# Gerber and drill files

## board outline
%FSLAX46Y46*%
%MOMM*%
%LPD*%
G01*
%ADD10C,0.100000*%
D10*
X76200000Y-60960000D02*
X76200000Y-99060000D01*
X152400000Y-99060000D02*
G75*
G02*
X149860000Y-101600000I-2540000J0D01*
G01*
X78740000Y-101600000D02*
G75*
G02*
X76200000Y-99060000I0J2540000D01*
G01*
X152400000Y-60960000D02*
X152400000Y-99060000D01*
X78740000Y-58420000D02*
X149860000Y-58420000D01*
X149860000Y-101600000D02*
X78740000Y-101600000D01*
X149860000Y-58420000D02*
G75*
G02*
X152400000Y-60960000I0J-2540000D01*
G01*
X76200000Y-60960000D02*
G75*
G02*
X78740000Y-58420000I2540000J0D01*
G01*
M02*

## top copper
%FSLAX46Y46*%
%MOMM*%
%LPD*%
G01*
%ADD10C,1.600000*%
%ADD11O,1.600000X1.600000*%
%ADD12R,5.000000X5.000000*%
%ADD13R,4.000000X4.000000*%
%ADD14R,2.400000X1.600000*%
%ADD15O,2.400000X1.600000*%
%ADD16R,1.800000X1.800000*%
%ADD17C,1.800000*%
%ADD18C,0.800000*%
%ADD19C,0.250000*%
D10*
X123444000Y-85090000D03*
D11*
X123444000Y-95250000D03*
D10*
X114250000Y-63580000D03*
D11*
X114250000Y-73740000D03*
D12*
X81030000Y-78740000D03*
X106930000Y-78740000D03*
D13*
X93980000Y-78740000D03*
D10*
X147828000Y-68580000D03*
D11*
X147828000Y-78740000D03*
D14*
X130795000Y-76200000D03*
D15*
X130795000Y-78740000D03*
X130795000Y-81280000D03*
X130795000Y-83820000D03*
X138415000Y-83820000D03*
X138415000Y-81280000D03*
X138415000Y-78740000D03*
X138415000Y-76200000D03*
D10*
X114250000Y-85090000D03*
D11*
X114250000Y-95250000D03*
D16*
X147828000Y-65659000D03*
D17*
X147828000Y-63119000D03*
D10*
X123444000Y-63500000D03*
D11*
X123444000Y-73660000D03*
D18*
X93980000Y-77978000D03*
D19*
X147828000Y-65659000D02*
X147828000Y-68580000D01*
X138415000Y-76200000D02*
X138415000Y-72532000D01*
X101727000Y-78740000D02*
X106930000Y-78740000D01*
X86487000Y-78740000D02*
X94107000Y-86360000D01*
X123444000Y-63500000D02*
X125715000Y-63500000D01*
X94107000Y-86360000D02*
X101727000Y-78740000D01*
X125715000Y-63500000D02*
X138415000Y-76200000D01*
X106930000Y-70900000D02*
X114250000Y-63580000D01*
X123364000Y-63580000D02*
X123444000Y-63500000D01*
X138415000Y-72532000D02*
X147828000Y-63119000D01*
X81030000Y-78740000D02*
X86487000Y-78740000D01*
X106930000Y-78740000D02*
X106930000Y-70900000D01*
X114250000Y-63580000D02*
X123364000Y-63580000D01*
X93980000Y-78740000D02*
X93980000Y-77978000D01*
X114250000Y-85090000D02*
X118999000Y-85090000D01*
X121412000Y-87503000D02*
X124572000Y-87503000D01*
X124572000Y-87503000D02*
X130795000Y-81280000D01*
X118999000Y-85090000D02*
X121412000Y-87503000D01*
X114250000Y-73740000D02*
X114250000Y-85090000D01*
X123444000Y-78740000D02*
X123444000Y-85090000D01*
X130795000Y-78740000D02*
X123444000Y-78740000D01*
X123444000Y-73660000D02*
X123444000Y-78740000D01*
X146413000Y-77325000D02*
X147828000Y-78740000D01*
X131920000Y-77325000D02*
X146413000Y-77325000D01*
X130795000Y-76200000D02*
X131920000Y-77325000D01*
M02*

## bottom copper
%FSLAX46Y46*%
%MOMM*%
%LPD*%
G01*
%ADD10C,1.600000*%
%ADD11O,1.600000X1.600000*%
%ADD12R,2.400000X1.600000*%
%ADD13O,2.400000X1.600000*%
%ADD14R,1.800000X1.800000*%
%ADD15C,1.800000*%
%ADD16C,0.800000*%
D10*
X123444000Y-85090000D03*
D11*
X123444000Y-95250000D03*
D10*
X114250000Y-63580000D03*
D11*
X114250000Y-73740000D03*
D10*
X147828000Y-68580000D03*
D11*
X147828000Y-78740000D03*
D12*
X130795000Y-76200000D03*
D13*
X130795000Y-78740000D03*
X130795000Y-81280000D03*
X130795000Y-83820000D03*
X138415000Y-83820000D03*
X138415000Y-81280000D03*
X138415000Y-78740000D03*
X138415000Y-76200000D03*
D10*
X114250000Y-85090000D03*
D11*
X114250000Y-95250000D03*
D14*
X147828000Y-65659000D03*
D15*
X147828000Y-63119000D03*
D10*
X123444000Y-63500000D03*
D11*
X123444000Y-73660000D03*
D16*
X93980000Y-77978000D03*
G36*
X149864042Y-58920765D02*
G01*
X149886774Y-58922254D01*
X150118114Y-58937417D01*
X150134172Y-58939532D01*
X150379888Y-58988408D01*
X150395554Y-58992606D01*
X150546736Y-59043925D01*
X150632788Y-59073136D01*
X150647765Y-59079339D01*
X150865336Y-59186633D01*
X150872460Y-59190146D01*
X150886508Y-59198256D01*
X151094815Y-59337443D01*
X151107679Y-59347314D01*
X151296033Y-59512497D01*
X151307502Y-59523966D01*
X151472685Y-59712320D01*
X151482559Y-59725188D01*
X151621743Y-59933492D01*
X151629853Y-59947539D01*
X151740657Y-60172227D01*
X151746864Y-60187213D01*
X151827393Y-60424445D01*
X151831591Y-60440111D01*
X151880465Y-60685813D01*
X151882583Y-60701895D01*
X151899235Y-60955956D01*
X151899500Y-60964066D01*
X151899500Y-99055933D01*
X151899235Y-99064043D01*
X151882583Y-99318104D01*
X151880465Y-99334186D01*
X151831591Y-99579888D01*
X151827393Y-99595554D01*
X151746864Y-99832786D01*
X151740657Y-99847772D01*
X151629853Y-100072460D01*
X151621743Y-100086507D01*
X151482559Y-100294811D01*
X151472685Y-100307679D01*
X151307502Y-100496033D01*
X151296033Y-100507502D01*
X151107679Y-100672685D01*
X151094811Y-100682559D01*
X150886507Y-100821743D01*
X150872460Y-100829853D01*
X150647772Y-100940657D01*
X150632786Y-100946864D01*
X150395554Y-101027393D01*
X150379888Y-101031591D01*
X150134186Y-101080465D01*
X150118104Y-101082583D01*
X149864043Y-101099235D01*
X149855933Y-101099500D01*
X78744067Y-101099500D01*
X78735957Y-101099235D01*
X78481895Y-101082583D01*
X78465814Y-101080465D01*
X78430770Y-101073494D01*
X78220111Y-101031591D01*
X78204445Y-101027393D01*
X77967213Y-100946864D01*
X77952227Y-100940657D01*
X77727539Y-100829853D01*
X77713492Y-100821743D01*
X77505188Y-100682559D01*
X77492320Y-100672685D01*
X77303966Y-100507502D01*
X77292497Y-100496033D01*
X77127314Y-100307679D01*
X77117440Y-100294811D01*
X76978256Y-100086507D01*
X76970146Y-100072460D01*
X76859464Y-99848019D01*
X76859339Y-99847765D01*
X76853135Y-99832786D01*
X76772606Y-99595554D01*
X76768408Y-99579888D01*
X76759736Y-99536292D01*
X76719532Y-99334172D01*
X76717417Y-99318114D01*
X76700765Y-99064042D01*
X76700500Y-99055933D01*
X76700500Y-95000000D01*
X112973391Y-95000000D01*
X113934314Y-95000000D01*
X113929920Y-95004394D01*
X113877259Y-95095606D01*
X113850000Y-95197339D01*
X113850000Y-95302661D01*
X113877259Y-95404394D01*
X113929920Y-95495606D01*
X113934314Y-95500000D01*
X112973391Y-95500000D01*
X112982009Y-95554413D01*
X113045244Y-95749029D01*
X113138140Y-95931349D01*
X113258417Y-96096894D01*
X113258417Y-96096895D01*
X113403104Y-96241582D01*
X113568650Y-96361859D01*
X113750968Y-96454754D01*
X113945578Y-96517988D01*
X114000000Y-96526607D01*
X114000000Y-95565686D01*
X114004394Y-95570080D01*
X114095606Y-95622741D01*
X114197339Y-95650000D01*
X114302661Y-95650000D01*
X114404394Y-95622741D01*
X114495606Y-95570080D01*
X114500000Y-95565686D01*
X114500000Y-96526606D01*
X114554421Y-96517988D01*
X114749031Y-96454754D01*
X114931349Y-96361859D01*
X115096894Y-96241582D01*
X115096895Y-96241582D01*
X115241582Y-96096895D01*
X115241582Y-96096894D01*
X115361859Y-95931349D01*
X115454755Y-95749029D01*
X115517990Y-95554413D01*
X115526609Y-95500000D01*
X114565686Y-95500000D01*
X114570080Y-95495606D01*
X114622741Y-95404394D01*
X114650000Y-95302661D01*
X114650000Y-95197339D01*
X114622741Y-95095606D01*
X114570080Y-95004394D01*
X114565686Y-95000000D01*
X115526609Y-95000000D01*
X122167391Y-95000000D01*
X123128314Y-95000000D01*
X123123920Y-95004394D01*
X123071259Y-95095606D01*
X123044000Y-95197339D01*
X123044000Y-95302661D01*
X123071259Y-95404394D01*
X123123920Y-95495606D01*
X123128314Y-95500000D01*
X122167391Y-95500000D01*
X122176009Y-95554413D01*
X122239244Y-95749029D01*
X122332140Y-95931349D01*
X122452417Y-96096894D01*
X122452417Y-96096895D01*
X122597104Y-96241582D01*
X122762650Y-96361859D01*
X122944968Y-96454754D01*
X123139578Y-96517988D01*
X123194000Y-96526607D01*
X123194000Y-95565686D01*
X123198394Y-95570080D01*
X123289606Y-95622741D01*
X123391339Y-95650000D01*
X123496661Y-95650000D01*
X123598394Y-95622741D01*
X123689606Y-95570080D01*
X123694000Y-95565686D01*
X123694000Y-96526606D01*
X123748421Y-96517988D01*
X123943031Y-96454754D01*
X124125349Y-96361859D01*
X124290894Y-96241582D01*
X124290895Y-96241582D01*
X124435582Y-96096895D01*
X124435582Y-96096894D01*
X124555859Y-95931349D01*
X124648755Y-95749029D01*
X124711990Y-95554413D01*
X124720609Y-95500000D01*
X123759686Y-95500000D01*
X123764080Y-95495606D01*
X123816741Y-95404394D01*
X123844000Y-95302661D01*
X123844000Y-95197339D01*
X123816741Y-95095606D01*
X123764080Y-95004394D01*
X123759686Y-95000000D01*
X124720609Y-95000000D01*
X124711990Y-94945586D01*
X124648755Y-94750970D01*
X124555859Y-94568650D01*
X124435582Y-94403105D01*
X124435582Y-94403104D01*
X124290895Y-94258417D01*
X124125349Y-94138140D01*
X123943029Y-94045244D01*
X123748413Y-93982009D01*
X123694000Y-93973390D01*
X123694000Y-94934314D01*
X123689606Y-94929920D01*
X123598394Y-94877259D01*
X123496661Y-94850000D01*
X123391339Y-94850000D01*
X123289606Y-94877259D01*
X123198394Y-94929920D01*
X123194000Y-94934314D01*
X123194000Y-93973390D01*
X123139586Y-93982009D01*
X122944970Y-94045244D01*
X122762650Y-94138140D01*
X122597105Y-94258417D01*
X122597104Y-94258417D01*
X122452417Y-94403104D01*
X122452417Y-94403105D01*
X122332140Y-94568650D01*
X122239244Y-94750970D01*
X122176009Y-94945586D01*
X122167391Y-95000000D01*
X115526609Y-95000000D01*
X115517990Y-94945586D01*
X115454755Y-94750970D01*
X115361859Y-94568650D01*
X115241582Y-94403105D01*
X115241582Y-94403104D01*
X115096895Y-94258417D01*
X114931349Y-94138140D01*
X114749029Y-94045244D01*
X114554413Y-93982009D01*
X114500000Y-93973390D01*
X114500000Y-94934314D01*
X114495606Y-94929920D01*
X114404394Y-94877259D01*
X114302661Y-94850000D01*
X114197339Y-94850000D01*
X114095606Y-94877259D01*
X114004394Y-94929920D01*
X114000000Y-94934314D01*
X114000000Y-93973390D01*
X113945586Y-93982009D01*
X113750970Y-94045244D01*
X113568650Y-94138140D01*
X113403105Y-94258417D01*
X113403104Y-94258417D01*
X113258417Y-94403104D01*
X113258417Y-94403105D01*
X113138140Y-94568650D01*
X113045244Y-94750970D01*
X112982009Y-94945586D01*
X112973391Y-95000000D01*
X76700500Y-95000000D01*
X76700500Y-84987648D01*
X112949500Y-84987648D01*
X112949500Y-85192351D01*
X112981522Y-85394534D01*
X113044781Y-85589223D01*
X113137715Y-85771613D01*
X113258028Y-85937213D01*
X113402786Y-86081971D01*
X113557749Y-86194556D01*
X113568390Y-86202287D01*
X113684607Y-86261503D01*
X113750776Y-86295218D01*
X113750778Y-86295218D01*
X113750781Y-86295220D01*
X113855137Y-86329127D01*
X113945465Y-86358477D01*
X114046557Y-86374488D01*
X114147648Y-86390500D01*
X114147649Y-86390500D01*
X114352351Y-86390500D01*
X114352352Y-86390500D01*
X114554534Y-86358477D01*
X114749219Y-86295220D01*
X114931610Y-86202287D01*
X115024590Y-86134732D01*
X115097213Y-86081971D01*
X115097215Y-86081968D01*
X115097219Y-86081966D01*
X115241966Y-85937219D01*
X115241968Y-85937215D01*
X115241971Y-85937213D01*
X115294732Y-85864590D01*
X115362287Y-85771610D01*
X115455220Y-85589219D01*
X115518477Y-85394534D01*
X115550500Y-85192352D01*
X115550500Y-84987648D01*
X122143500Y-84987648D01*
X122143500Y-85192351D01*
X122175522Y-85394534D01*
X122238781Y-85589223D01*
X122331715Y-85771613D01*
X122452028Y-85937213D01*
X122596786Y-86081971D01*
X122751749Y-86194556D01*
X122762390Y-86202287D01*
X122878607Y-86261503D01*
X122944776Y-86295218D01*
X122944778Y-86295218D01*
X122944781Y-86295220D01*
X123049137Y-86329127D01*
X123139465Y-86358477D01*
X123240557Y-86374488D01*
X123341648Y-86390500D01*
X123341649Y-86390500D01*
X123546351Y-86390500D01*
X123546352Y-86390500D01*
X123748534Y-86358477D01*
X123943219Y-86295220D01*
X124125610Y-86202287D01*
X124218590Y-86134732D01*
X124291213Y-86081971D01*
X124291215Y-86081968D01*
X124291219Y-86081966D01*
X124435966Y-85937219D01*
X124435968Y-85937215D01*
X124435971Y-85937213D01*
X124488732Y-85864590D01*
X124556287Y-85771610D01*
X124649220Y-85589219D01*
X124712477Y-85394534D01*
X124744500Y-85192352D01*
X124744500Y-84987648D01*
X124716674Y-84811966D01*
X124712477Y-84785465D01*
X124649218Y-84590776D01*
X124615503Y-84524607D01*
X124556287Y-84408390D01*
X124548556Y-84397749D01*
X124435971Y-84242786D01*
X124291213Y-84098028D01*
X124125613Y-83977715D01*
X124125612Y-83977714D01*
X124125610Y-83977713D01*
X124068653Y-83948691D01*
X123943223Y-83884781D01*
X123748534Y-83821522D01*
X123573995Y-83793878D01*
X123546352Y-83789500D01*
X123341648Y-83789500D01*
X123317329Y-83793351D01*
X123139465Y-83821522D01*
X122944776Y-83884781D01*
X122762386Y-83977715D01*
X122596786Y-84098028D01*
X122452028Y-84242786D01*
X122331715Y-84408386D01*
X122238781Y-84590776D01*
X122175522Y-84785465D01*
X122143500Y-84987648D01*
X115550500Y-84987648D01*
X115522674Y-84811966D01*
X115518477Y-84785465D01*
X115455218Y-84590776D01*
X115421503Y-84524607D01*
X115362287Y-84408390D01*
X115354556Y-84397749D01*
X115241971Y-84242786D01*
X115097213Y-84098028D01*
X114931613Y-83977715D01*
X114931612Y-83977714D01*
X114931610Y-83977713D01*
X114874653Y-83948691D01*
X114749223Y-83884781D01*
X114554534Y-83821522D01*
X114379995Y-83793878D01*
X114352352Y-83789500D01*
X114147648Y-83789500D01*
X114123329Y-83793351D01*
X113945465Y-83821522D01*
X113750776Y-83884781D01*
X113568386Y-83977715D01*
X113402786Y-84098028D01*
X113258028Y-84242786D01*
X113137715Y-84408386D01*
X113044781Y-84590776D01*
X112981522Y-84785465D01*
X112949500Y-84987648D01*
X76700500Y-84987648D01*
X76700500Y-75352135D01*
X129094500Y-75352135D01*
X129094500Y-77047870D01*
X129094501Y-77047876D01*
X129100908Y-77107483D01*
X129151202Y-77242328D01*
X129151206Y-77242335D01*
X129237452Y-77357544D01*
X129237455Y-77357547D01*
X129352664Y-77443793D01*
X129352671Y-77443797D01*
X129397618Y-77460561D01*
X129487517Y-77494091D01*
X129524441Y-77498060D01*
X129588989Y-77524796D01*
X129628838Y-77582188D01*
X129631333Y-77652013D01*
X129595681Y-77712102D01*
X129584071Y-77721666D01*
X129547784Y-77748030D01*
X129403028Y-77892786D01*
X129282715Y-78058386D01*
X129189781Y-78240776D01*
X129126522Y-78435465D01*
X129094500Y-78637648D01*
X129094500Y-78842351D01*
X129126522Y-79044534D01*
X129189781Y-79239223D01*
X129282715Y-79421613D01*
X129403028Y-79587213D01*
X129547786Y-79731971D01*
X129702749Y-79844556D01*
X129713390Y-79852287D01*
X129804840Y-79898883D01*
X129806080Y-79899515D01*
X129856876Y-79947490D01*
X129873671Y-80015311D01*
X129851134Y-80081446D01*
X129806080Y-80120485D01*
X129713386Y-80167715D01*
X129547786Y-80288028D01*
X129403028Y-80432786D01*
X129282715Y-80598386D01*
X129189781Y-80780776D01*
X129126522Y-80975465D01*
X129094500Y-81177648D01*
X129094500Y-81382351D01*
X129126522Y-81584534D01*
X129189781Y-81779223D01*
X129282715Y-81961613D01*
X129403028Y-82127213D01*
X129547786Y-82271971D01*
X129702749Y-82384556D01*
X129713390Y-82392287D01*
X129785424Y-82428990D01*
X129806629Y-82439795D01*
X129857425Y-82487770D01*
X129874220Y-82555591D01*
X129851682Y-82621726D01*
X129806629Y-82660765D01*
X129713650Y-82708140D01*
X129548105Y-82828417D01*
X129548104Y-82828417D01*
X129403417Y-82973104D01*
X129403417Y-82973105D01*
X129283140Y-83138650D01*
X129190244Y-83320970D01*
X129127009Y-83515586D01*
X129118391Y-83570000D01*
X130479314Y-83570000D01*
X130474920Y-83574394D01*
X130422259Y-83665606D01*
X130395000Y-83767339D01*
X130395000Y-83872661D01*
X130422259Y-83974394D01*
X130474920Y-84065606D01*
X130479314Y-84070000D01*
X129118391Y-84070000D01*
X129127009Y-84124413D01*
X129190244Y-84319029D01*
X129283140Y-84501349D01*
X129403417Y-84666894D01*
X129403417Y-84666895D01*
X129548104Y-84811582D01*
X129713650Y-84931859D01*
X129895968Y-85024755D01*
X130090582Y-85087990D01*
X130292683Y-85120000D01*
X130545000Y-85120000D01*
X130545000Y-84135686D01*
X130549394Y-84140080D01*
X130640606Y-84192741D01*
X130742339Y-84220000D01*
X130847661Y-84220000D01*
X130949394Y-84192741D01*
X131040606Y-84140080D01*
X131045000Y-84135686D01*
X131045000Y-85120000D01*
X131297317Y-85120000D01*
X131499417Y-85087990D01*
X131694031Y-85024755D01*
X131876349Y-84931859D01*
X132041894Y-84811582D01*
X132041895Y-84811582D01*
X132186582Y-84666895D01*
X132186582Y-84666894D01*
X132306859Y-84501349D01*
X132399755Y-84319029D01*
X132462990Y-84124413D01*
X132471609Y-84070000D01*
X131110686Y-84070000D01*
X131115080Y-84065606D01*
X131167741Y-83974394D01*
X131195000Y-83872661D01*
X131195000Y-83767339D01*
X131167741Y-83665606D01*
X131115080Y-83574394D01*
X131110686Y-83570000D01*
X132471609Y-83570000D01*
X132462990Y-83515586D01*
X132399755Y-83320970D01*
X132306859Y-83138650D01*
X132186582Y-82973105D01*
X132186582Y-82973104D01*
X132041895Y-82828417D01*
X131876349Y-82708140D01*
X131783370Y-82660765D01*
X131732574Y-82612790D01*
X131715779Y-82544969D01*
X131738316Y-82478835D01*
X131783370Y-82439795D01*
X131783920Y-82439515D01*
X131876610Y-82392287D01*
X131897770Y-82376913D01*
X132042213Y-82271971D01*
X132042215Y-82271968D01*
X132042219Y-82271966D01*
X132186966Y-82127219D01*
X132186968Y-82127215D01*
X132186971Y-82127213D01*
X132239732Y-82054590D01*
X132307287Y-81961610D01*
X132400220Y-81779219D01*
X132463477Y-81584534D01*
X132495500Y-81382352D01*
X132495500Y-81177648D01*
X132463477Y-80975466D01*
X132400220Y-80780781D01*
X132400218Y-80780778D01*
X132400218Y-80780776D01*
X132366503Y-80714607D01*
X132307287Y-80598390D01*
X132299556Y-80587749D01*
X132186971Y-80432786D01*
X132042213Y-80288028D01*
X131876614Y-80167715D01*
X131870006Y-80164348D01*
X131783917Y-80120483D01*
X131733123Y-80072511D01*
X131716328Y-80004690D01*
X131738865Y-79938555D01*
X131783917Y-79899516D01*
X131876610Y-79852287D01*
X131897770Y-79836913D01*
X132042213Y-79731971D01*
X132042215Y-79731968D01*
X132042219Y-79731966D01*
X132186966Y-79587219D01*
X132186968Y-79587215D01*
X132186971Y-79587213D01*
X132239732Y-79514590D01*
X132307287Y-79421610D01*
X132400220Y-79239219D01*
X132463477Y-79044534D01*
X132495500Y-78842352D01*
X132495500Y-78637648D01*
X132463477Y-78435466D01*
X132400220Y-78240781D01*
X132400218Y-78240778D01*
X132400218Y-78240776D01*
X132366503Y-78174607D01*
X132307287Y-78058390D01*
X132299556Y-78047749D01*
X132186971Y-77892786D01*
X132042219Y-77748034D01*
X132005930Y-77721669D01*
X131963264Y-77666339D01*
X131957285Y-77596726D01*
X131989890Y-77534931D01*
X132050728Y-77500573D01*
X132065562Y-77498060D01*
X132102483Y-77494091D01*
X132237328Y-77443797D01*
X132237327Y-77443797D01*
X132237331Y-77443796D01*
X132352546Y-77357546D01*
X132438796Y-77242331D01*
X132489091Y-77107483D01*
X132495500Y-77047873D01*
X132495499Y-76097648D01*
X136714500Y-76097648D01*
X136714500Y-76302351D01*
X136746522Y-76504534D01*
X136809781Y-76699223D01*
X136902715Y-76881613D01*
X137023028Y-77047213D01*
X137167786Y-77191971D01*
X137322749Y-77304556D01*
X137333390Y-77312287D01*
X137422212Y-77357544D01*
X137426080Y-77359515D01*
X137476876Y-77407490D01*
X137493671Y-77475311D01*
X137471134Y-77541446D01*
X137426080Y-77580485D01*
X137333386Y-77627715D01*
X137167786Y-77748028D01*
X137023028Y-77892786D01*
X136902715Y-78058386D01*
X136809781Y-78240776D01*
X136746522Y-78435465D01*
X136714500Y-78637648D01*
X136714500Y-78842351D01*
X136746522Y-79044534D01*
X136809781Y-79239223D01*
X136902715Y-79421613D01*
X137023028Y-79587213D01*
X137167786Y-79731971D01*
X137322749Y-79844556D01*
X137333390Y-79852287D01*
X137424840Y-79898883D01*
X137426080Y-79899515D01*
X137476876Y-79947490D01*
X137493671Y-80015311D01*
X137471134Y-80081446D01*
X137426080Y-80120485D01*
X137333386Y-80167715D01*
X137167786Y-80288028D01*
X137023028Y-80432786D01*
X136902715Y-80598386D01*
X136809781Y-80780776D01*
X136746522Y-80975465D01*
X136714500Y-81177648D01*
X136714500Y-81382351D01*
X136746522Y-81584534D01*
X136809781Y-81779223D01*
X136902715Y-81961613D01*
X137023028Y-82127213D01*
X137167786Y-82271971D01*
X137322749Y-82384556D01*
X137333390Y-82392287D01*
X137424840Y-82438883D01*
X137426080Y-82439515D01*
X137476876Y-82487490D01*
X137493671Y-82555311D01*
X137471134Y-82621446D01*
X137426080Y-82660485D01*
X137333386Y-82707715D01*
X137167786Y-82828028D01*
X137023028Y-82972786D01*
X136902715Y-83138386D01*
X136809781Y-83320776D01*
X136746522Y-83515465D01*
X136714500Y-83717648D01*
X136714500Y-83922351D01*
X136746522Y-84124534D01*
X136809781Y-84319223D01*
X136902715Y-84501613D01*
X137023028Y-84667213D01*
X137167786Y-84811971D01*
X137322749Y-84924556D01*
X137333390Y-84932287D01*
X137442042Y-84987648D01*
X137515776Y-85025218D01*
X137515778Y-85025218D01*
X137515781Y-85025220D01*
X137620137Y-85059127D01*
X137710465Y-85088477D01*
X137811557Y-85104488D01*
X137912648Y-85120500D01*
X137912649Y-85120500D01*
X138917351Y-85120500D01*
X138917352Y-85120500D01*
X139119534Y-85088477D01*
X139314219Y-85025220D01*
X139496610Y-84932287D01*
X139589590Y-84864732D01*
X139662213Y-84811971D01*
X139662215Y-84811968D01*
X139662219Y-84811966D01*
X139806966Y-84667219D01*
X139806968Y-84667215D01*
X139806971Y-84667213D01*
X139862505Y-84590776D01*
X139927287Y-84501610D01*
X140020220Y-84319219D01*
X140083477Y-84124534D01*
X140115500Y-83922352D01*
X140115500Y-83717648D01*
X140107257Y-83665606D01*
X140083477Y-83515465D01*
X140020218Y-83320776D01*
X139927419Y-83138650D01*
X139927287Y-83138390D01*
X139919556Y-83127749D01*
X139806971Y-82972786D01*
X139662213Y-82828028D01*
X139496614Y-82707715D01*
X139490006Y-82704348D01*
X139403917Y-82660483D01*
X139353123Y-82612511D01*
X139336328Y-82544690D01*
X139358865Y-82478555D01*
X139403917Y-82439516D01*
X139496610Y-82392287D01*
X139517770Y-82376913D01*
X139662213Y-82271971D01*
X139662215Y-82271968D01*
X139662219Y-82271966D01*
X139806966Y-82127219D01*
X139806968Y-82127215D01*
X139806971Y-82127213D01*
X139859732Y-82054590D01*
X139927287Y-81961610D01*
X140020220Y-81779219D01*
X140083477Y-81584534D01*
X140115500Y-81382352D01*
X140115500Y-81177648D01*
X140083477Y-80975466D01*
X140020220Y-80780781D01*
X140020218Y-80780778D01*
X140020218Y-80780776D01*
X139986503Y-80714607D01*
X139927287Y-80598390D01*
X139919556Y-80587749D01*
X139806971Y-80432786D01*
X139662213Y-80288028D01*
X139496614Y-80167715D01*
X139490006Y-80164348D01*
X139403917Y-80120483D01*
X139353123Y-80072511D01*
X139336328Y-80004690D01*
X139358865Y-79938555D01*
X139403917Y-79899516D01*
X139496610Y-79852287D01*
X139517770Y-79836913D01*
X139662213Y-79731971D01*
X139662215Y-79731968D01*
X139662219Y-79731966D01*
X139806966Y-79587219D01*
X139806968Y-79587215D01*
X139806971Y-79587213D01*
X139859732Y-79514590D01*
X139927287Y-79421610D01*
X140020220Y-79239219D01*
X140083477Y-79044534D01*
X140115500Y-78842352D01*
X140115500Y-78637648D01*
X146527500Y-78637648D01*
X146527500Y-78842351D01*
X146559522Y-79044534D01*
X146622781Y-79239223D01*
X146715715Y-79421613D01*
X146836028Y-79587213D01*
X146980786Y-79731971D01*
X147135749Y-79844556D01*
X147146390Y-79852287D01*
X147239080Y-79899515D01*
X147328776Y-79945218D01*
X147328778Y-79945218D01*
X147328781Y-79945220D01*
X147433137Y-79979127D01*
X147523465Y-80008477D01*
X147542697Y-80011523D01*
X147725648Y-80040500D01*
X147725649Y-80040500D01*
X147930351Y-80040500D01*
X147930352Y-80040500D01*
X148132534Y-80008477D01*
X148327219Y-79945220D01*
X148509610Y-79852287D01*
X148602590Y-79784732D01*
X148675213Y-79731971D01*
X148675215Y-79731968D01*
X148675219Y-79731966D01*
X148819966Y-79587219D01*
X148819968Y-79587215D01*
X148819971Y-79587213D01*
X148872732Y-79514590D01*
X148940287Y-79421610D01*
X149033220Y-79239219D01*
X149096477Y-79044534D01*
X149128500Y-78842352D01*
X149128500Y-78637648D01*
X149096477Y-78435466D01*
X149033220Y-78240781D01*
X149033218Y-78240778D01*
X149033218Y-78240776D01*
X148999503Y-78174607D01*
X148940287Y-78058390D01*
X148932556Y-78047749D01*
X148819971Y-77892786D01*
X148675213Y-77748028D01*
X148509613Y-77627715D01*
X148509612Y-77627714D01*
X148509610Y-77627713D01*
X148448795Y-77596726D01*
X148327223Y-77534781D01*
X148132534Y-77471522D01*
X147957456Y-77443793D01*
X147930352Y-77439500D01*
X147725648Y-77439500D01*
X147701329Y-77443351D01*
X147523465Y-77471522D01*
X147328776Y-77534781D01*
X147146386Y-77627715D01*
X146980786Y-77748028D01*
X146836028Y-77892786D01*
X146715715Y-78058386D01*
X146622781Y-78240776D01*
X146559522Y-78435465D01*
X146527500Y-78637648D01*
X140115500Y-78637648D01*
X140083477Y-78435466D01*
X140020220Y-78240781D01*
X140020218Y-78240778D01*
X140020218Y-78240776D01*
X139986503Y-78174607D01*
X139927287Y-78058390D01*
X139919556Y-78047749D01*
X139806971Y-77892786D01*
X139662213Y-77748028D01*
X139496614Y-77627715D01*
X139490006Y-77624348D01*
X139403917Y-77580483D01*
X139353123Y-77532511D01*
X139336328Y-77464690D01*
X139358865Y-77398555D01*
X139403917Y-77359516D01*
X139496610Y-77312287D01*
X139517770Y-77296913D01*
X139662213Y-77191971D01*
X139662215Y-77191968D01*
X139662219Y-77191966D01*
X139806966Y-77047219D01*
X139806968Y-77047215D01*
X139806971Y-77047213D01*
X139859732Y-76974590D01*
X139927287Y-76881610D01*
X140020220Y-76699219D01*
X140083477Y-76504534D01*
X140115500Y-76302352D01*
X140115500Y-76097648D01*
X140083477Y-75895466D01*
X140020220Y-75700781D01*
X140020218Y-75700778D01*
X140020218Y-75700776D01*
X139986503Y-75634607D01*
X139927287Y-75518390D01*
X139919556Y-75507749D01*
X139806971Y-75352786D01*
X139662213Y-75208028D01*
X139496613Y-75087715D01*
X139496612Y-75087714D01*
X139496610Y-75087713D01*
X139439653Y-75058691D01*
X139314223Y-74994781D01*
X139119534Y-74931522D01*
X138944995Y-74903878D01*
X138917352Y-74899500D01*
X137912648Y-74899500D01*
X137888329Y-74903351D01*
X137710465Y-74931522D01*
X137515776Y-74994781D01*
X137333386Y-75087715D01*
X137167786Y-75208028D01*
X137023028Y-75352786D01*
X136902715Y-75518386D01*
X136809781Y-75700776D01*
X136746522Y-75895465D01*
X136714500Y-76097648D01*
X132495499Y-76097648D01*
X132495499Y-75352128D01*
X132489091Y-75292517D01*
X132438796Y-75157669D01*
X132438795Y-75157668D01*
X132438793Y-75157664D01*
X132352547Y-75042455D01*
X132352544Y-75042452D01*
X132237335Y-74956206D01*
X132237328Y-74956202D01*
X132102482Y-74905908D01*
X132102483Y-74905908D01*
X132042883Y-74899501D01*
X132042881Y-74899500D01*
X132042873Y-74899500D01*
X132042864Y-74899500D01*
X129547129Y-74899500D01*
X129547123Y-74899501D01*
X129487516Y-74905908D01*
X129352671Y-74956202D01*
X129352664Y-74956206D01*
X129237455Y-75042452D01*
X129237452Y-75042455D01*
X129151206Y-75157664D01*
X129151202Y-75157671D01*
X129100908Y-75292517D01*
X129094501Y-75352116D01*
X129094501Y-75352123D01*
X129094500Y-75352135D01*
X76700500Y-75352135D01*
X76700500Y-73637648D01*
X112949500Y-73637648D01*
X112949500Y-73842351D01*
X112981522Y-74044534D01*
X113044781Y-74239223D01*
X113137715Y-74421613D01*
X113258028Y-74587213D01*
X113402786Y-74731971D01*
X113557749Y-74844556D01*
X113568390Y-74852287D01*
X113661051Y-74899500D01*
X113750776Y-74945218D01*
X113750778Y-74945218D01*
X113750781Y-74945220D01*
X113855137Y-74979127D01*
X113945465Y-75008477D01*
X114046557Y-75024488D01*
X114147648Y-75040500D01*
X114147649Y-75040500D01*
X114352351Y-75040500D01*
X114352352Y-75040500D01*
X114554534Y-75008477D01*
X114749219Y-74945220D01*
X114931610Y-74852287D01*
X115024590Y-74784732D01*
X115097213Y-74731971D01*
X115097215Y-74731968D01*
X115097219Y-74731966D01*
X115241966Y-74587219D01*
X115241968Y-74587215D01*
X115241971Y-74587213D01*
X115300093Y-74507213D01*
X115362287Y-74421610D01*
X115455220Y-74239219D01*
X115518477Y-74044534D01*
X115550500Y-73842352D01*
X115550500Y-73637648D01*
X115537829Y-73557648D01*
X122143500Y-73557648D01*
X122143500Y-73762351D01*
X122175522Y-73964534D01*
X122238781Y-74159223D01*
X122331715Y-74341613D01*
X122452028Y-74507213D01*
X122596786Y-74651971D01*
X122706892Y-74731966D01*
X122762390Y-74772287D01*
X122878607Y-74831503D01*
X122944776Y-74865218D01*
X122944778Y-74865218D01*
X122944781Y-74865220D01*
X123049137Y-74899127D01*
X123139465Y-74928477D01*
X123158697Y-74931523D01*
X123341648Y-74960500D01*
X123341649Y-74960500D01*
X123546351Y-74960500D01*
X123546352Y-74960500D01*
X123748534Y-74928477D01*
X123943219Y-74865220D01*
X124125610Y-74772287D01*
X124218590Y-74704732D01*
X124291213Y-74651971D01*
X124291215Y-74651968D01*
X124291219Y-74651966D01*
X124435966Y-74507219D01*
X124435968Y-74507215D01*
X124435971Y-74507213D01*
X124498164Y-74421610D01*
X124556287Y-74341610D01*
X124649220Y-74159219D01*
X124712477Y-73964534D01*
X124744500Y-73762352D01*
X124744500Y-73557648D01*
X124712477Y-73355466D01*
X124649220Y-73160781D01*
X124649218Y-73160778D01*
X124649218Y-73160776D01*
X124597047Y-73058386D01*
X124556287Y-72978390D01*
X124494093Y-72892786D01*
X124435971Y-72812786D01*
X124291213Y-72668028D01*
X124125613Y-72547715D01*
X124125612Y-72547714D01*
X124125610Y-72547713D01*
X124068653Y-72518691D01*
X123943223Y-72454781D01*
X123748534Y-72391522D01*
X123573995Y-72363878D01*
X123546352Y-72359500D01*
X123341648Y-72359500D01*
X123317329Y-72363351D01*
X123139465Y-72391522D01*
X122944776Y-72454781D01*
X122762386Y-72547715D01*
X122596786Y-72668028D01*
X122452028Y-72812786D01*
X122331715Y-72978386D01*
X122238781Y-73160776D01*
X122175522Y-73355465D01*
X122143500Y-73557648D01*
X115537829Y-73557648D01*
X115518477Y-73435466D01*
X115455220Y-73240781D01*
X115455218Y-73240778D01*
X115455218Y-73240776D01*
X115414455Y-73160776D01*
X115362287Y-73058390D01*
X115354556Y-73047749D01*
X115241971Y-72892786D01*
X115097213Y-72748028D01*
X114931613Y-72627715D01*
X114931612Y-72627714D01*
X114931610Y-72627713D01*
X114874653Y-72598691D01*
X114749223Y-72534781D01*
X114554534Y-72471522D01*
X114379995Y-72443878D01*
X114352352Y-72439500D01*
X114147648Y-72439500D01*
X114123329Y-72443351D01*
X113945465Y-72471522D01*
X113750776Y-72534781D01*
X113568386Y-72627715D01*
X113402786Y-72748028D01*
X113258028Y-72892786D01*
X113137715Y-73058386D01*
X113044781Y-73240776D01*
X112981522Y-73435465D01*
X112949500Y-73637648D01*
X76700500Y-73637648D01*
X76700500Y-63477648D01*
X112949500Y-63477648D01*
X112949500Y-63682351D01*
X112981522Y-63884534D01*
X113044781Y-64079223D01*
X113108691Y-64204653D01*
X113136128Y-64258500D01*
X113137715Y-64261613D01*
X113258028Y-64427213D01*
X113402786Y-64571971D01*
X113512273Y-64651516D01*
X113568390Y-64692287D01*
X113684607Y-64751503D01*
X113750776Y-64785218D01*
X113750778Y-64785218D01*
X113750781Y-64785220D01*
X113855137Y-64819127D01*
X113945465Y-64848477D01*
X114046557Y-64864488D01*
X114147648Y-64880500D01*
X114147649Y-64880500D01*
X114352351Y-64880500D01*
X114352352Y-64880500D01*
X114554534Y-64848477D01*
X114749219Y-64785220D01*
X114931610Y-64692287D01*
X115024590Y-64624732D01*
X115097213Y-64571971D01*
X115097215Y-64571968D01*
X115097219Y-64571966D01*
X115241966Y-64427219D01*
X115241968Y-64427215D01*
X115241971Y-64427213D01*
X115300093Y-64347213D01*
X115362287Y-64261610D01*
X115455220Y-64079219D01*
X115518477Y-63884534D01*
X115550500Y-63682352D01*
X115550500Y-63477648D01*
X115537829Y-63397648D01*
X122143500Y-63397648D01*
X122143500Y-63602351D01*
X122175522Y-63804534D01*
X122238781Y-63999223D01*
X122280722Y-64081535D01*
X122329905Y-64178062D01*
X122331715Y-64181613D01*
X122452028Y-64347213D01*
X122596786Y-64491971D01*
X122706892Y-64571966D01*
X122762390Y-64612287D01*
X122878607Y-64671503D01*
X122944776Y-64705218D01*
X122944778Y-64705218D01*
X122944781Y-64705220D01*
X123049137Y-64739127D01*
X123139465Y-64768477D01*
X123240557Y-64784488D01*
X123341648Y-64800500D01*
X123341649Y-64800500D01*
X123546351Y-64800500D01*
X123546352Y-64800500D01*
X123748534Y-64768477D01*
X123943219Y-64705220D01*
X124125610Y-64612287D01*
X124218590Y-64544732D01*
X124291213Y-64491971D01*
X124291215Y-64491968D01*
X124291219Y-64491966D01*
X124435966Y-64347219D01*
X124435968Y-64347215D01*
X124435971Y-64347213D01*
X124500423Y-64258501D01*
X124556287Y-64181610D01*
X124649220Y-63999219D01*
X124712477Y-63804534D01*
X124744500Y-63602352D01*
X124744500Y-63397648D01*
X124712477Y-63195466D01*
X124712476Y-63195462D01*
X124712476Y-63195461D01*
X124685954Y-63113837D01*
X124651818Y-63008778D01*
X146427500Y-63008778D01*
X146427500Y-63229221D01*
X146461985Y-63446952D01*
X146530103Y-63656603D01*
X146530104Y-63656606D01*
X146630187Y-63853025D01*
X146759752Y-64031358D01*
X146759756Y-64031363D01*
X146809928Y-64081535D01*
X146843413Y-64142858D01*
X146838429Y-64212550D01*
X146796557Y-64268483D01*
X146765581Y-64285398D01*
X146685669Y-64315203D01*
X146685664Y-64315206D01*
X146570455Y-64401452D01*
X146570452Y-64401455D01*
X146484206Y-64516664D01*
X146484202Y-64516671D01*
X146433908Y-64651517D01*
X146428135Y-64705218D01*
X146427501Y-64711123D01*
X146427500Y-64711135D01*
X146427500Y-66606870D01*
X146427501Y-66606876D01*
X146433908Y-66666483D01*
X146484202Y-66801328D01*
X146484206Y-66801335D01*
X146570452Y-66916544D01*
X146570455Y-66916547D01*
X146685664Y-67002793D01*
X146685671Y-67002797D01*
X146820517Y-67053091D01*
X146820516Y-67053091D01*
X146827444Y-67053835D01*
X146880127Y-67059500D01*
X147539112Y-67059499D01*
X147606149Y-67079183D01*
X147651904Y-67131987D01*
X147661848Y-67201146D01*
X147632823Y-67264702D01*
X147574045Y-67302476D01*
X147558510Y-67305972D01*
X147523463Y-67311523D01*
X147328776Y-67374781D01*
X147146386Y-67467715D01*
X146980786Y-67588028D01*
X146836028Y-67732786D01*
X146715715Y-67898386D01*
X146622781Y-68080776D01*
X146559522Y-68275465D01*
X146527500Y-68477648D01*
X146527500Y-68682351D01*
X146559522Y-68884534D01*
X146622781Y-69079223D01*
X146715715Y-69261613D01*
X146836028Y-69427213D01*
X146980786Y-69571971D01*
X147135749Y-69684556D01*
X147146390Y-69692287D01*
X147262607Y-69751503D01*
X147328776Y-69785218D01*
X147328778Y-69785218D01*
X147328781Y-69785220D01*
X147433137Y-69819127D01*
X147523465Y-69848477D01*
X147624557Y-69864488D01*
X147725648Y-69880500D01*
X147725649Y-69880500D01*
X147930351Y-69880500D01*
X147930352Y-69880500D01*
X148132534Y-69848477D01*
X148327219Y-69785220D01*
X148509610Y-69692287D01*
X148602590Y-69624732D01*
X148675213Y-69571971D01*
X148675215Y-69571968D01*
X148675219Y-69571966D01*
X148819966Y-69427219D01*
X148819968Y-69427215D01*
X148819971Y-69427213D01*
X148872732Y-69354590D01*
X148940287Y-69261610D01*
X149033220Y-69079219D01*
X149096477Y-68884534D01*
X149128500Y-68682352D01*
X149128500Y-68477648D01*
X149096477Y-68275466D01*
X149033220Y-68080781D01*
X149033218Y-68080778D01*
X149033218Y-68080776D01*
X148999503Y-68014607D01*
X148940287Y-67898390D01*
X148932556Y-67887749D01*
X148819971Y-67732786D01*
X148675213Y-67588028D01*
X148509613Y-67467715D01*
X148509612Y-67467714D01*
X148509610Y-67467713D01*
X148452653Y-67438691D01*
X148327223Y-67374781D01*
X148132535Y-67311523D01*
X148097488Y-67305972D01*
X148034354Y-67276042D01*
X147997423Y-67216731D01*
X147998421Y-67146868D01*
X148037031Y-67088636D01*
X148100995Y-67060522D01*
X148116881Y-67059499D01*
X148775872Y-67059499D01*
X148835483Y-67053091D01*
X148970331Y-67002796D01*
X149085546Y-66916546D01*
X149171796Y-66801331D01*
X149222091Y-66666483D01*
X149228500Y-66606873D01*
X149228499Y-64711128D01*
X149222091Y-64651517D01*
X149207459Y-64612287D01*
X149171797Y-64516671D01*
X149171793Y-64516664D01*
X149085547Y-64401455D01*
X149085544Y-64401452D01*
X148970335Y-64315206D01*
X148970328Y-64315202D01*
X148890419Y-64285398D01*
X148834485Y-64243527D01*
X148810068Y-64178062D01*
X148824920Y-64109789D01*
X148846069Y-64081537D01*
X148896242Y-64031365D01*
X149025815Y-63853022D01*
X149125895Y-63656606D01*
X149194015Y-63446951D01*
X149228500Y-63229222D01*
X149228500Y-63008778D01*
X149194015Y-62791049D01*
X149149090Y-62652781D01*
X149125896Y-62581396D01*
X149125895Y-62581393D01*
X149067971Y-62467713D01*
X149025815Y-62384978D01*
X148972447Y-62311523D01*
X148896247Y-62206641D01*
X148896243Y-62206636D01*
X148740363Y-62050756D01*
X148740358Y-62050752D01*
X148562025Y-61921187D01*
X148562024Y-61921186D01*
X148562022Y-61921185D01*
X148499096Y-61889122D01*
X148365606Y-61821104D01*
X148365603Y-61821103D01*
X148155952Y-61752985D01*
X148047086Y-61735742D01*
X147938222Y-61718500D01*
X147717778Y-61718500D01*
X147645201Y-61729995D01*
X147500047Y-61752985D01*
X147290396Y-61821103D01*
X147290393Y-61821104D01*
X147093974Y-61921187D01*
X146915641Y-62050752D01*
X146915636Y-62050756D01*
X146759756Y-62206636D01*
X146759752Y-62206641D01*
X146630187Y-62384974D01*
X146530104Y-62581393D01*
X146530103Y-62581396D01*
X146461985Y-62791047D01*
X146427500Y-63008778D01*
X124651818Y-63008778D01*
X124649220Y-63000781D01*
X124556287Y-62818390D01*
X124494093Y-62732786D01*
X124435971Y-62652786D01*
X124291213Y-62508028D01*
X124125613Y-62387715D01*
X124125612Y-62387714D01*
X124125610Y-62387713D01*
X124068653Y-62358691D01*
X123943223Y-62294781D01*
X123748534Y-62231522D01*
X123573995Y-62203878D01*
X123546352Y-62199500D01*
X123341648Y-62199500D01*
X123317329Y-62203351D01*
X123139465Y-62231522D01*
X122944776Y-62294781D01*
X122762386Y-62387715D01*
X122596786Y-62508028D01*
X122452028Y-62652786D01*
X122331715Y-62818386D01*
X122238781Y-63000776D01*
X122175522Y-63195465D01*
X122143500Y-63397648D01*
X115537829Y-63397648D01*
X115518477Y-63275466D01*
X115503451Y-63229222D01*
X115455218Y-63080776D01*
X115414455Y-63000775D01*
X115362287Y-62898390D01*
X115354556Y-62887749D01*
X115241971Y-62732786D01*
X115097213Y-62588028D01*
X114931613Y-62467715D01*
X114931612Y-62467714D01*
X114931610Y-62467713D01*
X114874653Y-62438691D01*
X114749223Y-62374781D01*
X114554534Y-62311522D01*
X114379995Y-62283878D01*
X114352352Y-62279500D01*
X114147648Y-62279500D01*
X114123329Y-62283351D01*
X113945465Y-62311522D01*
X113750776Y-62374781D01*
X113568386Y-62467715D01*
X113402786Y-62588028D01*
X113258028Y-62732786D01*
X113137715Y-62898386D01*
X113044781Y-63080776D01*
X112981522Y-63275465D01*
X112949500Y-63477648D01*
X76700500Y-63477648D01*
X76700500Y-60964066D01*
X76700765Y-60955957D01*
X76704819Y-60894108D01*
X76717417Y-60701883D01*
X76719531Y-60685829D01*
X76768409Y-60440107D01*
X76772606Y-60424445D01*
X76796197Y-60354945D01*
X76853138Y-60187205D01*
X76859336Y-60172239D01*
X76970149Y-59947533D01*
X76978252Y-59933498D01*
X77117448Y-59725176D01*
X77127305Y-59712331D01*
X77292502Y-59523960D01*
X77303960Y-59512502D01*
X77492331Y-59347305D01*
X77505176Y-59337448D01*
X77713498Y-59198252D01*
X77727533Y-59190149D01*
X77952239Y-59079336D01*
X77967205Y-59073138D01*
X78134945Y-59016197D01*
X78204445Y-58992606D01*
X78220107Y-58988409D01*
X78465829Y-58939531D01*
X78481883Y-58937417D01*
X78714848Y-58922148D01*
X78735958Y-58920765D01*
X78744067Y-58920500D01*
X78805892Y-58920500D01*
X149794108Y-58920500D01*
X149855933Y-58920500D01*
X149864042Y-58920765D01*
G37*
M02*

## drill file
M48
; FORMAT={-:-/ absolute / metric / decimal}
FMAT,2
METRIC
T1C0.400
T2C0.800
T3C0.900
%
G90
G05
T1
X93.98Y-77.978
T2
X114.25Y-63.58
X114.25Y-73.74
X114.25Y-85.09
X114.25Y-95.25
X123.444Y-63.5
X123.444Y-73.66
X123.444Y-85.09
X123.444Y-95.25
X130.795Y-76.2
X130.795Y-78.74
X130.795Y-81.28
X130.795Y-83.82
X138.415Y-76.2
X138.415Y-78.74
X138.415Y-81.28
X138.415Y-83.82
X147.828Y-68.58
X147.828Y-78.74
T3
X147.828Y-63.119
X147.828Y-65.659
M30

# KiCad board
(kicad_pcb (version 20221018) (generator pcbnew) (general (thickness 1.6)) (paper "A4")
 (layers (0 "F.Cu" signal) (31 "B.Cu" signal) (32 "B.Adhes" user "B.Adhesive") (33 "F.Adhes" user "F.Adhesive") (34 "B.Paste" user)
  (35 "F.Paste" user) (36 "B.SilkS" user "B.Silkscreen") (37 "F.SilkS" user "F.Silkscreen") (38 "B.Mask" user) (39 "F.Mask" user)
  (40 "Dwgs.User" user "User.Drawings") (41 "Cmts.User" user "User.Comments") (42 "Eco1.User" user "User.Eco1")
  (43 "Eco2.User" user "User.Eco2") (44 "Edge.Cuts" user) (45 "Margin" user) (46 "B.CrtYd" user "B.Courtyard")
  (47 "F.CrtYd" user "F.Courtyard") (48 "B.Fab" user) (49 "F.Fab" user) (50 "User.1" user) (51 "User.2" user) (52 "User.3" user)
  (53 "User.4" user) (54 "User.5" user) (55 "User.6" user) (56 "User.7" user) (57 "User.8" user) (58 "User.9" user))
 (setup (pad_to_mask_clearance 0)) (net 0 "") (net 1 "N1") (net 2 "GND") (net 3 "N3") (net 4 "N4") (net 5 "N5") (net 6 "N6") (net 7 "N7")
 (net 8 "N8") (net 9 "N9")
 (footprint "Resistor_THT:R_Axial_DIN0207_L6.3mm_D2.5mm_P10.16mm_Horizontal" (layer "F.Cu") (at 123.444 85.09 -90)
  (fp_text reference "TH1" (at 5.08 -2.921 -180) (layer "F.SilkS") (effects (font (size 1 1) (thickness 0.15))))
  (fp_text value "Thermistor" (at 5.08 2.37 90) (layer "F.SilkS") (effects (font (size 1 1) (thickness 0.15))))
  (pad "1" thru_hole circle (at 0 0 270) (size 1.6 1.6) (drill 0.8) (layers "*.Cu" "*.Mask") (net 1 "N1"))
  (pad "2" thru_hole oval (at 10.16 0 270) (size 1.6 1.6) (drill 0.8) (layers "*.Cu" "*.Mask") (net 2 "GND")))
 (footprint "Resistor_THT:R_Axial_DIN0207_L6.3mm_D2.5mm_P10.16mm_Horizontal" (layer "F.Cu") (at 114.25 63.58 -90)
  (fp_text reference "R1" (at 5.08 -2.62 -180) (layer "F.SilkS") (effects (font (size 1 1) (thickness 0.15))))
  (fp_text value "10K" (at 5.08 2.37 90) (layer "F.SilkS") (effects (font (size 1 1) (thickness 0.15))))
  (pad "1" thru_hole circle (at 0 0 270) (size 1.6 1.6) (drill 0.8) (layers "*.Cu" "*.Mask") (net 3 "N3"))
  (pad "2" thru_hole oval (at 10.16 0 270) (size 1.6 1.6) (drill 0.8) (layers "*.Cu" "*.Mask") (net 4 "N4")))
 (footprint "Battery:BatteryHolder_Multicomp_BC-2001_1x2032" (layer "F.Cu") (at 93.98 78.74)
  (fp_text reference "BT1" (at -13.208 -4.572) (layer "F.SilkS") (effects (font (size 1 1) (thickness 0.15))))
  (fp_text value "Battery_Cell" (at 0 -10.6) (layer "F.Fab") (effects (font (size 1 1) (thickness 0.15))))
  (pad "1" smd rect (at -12.95 0) (size 5 5) (layers "F.Cu" "F.Paste" "F.Mask") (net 3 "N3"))
  (pad "1" smd rect (at 12.95 0) (size 5 5) (layers "F.Cu" "F.Paste" "F.Mask") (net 3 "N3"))
  (pad "2" smd rect (at 0 0) (size 4 4) (layers "F.Cu" "F.Paste" "F.Mask") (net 2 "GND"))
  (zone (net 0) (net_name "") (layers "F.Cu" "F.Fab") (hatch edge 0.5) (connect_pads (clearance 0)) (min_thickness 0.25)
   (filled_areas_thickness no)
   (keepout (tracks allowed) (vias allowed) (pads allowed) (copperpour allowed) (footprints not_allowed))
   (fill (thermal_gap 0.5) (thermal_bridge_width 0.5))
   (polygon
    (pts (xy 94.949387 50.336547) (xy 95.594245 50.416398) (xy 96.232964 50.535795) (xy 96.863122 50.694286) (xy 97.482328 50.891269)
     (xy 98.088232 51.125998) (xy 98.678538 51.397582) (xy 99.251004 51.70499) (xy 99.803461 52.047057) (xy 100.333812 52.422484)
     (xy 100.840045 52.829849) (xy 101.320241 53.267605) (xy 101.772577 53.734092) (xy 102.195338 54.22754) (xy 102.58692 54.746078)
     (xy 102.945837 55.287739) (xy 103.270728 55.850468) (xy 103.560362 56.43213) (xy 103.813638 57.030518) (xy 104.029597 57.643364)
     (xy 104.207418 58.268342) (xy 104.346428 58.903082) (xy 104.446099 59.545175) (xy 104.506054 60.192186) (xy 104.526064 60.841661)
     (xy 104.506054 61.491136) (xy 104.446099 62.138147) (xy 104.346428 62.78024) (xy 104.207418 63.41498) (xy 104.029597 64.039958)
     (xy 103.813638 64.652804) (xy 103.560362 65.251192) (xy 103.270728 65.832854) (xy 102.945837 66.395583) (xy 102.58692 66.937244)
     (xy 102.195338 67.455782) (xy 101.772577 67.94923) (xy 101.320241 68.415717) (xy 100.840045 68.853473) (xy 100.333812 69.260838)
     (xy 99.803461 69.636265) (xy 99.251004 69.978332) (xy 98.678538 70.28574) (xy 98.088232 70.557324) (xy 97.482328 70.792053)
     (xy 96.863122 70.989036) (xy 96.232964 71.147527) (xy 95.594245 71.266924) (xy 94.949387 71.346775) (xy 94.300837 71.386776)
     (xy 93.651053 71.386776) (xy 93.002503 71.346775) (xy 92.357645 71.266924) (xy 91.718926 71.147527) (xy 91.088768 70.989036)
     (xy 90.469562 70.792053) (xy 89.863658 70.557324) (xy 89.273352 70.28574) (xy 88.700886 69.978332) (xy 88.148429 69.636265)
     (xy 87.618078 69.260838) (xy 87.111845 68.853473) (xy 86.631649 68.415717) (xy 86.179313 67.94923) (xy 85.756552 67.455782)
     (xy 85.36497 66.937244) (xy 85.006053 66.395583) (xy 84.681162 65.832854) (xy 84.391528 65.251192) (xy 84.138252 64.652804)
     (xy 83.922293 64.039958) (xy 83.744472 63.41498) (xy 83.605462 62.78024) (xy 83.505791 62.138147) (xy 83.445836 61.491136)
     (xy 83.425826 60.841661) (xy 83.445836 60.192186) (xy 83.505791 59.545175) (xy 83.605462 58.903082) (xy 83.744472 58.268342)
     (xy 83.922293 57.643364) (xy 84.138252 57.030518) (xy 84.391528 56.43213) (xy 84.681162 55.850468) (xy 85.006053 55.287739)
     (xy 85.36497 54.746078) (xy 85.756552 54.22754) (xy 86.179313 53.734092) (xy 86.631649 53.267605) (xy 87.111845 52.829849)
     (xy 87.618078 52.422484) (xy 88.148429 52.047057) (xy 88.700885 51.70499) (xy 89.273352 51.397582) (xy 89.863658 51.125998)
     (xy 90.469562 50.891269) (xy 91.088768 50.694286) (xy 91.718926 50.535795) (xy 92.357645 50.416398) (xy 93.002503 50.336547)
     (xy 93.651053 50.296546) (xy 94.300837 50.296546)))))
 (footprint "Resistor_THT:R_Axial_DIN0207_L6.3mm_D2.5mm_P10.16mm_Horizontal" (layer "F.Cu") (at 147.828 68.58 -90)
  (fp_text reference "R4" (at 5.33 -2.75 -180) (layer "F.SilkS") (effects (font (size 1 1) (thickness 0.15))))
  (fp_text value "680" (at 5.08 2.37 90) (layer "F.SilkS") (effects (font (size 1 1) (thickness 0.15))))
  (pad "1" thru_hole circle (at 0 0 270) (size 1.6 1.6) (drill 0.8) (layers "*.Cu" "*.Mask") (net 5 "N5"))
  (pad "2" thru_hole oval (at 10.16 0 270) (size 1.6 1.6) (drill 0.8) (layers "*.Cu" "*.Mask") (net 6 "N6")))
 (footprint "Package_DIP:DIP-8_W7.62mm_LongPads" (layer "F.Cu") (at 130.795 76.2)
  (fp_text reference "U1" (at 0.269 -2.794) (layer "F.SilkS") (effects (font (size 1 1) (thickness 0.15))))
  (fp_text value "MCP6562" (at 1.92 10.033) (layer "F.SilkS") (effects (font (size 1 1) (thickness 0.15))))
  (pad "1" thru_hole rect (at 0 0) (size 2.4 1.6) (drill 0.8) (layers "*.Cu" "*.Mask") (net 6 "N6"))
  (pad "2" thru_hole oval (at 0 2.54) (size 2.4 1.6) (drill 0.8) (layers "*.Cu" "*.Mask") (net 1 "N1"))
  (pad "3" thru_hole oval (at 0 5.08) (size 2.4 1.6) (drill 0.8) (layers "*.Cu" "*.Mask") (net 4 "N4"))
  (pad "4" thru_hole oval (at 0 7.62) (size 2.4 1.6) (drill 0.8) (layers "*.Cu" "*.Mask") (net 2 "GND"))
  (pad "5" thru_hole oval (at 7.62 7.62) (size 2.4 1.6) (drill 0.8) (layers "*.Cu" "*.Mask") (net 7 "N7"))
  (pad "6" thru_hole oval (at 7.62 5.08) (size 2.4 1.6) (drill 0.8) (layers "*.Cu" "*.Mask") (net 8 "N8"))
  (pad "7" thru_hole oval (at 7.62 2.54) (size 2.4 1.6) (drill 0.8) (layers "*.Cu" "*.Mask") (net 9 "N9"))
  (pad "8" thru_hole oval (at 7.62 0) (size 2.4 1.6) (drill 0.8) (layers "*.Cu" "*.Mask") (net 3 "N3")))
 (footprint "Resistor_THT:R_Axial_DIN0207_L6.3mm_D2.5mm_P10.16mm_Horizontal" (layer "F.Cu") (at 114.25 85.09 -90)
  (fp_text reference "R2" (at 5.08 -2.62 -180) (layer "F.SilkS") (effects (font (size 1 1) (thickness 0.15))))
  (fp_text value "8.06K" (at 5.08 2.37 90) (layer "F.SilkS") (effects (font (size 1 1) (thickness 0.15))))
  (pad "1" thru_hole circle (at 0 0 270) (size 1.6 1.6) (drill 0.8) (layers "*.Cu" "*.Mask") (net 4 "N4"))
  (pad "2" thru_hole oval (at 10.16 0 270) (size 1.6 1.6) (drill 0.8) (layers "*.Cu" "*.Mask") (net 2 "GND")))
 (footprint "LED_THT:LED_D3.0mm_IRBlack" (layer "F.Cu") (at 147.828 65.659 90)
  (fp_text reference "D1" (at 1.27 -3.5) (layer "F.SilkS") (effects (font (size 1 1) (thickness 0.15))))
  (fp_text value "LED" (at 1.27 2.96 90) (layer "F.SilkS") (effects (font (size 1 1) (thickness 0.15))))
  (pad "1" thru_hole rect (at 0 0 90) (size 1.8 1.8) (drill 0.9) (layers "*.Cu" "*.Mask") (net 5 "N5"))
  (pad "2" thru_hole circle (at 2.54 0 90) (size 1.8 1.8) (drill 0.9) (layers "*.Cu" "*.Mask") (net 3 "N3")))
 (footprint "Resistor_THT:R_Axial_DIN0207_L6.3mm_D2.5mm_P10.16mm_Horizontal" (layer "F.Cu") (at 123.444 63.5 -90)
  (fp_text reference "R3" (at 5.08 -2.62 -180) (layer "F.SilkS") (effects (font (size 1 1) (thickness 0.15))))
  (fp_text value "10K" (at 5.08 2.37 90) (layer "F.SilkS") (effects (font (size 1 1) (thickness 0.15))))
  (pad "1" thru_hole circle (at 0 0 270) (size 1.6 1.6) (drill 0.8) (layers "*.Cu" "*.Mask") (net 3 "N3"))
  (pad "2" thru_hole oval (at 10.16 0 270) (size 1.6 1.6) (drill 0.8) (layers "*.Cu" "*.Mask") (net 1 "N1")))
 (gr_line (start 76.2 60.96) (end 76.2 99.06) (stroke (width 0.1) (type default)) (layer "Edge.Cuts"))
 (gr_arc (start 152.4 99.06) (mid 151.656051 100.856051) (end 149.86 101.6) (stroke (width 0.1) (type default)) (layer "Edge.Cuts"))
 (gr_arc (start 78.74 101.6) (mid 76.943949 100.856051) (end 76.2 99.06) (stroke (width 0.1) (type default)) (layer "Edge.Cuts"))
 (gr_line (start 152.4 60.96) (end 152.4 99.06) (stroke (width 0.1) (type default)) (layer "Edge.Cuts"))
 (gr_line (start 78.74 58.42) (end 149.86 58.42) (stroke (width 0.1) (type default)) (layer "Edge.Cuts"))
 (gr_line (start 149.86 101.6) (end 78.74 101.6) (stroke (width 0.1) (type default)) (layer "Edge.Cuts"))
 (gr_arc (start 149.86 58.42) (mid 151.656051 59.163949) (end 152.4 60.96) (stroke (width 0.1) (type default)) (layer "Edge.Cuts"))
 (gr_arc (start 76.2 60.96) (mid 76.943949 59.163949) (end 78.74 58.42) (stroke (width 0.1) (type default)) (layer "Edge.Cuts"))
 (segment (start 147.828 65.659) (end 147.828 68.58) (width 0.25) (layer "F.Cu") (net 5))
 (segment (start 138.415 76.2) (end 138.415 72.532) (width 0.25) (layer "F.Cu") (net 3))
 (segment (start 101.727 78.74) (end 106.93 78.74) (width 0.25) (layer "F.Cu") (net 3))
 (segment (start 86.487 78.74) (end 94.107 86.36) (width 0.25) (layer "F.Cu") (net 3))
 (segment (start 123.444 63.5) (end 125.715 63.5) (width 0.25) (layer "F.Cu") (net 3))
 (segment (start 94.107 86.36) (end 101.727 78.74) (width 0.25) (layer "F.Cu") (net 3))
 (segment (start 125.715 63.5) (end 138.415 76.2) (width 0.25) (layer "F.Cu") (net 3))
 (segment (start 106.93 70.9) (end 114.25 63.58) (width 0.25) (layer "F.Cu") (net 3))
 (segment (start 123.364 63.58) (end 123.444 63.5) (width 0.25) (layer "F.Cu") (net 3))
 (segment (start 138.415 72.532) (end 147.828 63.119) (width 0.25) (layer "F.Cu") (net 3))
 (segment (start 81.03 78.74) (end 86.487 78.74) (width 0.25) (layer "F.Cu") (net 3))
 (segment (start 106.93 78.74) (end 106.93 70.9) (width 0.25) (layer "F.Cu") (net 3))
 (segment (start 114.25 63.58) (end 123.364 63.58) (width 0.25) (layer "F.Cu") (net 3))
 (segment (start 93.98 78.74) (end 93.98 77.978) (width 0.25) (layer "F.Cu") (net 2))
 (via (at 93.98 77.978) (size 0.8) (drill 0.4) (layers "F.Cu" "B.Cu") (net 2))
 (segment (start 114.25 85.09) (end 118.999 85.09) (width 0.25) (layer "F.Cu") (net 4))
 (segment (start 121.412 87.503) (end 124.572 87.503) (width 0.25) (layer "F.Cu") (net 4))
 (segment (start 124.572 87.503) (end 130.795 81.28) (width 0.25) (layer "F.Cu") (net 4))
 (segment (start 118.999 85.09) (end 121.412 87.503) (width 0.25) (layer "F.Cu") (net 4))
 (segment (start 114.25 73.74) (end 114.25 85.09) (width 0.25) (layer "F.Cu") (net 4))
 (segment (start 123.444 78.74) (end 123.444 85.09) (width 0.25) (layer "F.Cu") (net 1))
 (segment (start 130.795 78.74) (end 123.444 78.74) (width 0.25) (layer "F.Cu") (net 1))
 (segment (start 123.444 73.66) (end 123.444 78.74) (width 0.25) (layer "F.Cu") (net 1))
 (segment (start 146.413 77.325) (end 147.828 78.74) (width 0.25) (layer "F.Cu") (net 6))
 (segment (start 131.92 77.325) (end 146.413 77.325) (width 0.25) (layer "F.Cu") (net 6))
 (segment (start 130.795 76.2) (end 131.92 77.325) (width 0.25) (layer "F.Cu") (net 6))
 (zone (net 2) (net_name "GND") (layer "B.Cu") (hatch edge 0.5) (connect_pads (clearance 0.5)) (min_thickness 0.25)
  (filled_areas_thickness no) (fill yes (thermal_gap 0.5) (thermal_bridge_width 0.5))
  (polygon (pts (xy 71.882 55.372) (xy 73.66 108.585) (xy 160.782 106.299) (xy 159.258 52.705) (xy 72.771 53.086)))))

